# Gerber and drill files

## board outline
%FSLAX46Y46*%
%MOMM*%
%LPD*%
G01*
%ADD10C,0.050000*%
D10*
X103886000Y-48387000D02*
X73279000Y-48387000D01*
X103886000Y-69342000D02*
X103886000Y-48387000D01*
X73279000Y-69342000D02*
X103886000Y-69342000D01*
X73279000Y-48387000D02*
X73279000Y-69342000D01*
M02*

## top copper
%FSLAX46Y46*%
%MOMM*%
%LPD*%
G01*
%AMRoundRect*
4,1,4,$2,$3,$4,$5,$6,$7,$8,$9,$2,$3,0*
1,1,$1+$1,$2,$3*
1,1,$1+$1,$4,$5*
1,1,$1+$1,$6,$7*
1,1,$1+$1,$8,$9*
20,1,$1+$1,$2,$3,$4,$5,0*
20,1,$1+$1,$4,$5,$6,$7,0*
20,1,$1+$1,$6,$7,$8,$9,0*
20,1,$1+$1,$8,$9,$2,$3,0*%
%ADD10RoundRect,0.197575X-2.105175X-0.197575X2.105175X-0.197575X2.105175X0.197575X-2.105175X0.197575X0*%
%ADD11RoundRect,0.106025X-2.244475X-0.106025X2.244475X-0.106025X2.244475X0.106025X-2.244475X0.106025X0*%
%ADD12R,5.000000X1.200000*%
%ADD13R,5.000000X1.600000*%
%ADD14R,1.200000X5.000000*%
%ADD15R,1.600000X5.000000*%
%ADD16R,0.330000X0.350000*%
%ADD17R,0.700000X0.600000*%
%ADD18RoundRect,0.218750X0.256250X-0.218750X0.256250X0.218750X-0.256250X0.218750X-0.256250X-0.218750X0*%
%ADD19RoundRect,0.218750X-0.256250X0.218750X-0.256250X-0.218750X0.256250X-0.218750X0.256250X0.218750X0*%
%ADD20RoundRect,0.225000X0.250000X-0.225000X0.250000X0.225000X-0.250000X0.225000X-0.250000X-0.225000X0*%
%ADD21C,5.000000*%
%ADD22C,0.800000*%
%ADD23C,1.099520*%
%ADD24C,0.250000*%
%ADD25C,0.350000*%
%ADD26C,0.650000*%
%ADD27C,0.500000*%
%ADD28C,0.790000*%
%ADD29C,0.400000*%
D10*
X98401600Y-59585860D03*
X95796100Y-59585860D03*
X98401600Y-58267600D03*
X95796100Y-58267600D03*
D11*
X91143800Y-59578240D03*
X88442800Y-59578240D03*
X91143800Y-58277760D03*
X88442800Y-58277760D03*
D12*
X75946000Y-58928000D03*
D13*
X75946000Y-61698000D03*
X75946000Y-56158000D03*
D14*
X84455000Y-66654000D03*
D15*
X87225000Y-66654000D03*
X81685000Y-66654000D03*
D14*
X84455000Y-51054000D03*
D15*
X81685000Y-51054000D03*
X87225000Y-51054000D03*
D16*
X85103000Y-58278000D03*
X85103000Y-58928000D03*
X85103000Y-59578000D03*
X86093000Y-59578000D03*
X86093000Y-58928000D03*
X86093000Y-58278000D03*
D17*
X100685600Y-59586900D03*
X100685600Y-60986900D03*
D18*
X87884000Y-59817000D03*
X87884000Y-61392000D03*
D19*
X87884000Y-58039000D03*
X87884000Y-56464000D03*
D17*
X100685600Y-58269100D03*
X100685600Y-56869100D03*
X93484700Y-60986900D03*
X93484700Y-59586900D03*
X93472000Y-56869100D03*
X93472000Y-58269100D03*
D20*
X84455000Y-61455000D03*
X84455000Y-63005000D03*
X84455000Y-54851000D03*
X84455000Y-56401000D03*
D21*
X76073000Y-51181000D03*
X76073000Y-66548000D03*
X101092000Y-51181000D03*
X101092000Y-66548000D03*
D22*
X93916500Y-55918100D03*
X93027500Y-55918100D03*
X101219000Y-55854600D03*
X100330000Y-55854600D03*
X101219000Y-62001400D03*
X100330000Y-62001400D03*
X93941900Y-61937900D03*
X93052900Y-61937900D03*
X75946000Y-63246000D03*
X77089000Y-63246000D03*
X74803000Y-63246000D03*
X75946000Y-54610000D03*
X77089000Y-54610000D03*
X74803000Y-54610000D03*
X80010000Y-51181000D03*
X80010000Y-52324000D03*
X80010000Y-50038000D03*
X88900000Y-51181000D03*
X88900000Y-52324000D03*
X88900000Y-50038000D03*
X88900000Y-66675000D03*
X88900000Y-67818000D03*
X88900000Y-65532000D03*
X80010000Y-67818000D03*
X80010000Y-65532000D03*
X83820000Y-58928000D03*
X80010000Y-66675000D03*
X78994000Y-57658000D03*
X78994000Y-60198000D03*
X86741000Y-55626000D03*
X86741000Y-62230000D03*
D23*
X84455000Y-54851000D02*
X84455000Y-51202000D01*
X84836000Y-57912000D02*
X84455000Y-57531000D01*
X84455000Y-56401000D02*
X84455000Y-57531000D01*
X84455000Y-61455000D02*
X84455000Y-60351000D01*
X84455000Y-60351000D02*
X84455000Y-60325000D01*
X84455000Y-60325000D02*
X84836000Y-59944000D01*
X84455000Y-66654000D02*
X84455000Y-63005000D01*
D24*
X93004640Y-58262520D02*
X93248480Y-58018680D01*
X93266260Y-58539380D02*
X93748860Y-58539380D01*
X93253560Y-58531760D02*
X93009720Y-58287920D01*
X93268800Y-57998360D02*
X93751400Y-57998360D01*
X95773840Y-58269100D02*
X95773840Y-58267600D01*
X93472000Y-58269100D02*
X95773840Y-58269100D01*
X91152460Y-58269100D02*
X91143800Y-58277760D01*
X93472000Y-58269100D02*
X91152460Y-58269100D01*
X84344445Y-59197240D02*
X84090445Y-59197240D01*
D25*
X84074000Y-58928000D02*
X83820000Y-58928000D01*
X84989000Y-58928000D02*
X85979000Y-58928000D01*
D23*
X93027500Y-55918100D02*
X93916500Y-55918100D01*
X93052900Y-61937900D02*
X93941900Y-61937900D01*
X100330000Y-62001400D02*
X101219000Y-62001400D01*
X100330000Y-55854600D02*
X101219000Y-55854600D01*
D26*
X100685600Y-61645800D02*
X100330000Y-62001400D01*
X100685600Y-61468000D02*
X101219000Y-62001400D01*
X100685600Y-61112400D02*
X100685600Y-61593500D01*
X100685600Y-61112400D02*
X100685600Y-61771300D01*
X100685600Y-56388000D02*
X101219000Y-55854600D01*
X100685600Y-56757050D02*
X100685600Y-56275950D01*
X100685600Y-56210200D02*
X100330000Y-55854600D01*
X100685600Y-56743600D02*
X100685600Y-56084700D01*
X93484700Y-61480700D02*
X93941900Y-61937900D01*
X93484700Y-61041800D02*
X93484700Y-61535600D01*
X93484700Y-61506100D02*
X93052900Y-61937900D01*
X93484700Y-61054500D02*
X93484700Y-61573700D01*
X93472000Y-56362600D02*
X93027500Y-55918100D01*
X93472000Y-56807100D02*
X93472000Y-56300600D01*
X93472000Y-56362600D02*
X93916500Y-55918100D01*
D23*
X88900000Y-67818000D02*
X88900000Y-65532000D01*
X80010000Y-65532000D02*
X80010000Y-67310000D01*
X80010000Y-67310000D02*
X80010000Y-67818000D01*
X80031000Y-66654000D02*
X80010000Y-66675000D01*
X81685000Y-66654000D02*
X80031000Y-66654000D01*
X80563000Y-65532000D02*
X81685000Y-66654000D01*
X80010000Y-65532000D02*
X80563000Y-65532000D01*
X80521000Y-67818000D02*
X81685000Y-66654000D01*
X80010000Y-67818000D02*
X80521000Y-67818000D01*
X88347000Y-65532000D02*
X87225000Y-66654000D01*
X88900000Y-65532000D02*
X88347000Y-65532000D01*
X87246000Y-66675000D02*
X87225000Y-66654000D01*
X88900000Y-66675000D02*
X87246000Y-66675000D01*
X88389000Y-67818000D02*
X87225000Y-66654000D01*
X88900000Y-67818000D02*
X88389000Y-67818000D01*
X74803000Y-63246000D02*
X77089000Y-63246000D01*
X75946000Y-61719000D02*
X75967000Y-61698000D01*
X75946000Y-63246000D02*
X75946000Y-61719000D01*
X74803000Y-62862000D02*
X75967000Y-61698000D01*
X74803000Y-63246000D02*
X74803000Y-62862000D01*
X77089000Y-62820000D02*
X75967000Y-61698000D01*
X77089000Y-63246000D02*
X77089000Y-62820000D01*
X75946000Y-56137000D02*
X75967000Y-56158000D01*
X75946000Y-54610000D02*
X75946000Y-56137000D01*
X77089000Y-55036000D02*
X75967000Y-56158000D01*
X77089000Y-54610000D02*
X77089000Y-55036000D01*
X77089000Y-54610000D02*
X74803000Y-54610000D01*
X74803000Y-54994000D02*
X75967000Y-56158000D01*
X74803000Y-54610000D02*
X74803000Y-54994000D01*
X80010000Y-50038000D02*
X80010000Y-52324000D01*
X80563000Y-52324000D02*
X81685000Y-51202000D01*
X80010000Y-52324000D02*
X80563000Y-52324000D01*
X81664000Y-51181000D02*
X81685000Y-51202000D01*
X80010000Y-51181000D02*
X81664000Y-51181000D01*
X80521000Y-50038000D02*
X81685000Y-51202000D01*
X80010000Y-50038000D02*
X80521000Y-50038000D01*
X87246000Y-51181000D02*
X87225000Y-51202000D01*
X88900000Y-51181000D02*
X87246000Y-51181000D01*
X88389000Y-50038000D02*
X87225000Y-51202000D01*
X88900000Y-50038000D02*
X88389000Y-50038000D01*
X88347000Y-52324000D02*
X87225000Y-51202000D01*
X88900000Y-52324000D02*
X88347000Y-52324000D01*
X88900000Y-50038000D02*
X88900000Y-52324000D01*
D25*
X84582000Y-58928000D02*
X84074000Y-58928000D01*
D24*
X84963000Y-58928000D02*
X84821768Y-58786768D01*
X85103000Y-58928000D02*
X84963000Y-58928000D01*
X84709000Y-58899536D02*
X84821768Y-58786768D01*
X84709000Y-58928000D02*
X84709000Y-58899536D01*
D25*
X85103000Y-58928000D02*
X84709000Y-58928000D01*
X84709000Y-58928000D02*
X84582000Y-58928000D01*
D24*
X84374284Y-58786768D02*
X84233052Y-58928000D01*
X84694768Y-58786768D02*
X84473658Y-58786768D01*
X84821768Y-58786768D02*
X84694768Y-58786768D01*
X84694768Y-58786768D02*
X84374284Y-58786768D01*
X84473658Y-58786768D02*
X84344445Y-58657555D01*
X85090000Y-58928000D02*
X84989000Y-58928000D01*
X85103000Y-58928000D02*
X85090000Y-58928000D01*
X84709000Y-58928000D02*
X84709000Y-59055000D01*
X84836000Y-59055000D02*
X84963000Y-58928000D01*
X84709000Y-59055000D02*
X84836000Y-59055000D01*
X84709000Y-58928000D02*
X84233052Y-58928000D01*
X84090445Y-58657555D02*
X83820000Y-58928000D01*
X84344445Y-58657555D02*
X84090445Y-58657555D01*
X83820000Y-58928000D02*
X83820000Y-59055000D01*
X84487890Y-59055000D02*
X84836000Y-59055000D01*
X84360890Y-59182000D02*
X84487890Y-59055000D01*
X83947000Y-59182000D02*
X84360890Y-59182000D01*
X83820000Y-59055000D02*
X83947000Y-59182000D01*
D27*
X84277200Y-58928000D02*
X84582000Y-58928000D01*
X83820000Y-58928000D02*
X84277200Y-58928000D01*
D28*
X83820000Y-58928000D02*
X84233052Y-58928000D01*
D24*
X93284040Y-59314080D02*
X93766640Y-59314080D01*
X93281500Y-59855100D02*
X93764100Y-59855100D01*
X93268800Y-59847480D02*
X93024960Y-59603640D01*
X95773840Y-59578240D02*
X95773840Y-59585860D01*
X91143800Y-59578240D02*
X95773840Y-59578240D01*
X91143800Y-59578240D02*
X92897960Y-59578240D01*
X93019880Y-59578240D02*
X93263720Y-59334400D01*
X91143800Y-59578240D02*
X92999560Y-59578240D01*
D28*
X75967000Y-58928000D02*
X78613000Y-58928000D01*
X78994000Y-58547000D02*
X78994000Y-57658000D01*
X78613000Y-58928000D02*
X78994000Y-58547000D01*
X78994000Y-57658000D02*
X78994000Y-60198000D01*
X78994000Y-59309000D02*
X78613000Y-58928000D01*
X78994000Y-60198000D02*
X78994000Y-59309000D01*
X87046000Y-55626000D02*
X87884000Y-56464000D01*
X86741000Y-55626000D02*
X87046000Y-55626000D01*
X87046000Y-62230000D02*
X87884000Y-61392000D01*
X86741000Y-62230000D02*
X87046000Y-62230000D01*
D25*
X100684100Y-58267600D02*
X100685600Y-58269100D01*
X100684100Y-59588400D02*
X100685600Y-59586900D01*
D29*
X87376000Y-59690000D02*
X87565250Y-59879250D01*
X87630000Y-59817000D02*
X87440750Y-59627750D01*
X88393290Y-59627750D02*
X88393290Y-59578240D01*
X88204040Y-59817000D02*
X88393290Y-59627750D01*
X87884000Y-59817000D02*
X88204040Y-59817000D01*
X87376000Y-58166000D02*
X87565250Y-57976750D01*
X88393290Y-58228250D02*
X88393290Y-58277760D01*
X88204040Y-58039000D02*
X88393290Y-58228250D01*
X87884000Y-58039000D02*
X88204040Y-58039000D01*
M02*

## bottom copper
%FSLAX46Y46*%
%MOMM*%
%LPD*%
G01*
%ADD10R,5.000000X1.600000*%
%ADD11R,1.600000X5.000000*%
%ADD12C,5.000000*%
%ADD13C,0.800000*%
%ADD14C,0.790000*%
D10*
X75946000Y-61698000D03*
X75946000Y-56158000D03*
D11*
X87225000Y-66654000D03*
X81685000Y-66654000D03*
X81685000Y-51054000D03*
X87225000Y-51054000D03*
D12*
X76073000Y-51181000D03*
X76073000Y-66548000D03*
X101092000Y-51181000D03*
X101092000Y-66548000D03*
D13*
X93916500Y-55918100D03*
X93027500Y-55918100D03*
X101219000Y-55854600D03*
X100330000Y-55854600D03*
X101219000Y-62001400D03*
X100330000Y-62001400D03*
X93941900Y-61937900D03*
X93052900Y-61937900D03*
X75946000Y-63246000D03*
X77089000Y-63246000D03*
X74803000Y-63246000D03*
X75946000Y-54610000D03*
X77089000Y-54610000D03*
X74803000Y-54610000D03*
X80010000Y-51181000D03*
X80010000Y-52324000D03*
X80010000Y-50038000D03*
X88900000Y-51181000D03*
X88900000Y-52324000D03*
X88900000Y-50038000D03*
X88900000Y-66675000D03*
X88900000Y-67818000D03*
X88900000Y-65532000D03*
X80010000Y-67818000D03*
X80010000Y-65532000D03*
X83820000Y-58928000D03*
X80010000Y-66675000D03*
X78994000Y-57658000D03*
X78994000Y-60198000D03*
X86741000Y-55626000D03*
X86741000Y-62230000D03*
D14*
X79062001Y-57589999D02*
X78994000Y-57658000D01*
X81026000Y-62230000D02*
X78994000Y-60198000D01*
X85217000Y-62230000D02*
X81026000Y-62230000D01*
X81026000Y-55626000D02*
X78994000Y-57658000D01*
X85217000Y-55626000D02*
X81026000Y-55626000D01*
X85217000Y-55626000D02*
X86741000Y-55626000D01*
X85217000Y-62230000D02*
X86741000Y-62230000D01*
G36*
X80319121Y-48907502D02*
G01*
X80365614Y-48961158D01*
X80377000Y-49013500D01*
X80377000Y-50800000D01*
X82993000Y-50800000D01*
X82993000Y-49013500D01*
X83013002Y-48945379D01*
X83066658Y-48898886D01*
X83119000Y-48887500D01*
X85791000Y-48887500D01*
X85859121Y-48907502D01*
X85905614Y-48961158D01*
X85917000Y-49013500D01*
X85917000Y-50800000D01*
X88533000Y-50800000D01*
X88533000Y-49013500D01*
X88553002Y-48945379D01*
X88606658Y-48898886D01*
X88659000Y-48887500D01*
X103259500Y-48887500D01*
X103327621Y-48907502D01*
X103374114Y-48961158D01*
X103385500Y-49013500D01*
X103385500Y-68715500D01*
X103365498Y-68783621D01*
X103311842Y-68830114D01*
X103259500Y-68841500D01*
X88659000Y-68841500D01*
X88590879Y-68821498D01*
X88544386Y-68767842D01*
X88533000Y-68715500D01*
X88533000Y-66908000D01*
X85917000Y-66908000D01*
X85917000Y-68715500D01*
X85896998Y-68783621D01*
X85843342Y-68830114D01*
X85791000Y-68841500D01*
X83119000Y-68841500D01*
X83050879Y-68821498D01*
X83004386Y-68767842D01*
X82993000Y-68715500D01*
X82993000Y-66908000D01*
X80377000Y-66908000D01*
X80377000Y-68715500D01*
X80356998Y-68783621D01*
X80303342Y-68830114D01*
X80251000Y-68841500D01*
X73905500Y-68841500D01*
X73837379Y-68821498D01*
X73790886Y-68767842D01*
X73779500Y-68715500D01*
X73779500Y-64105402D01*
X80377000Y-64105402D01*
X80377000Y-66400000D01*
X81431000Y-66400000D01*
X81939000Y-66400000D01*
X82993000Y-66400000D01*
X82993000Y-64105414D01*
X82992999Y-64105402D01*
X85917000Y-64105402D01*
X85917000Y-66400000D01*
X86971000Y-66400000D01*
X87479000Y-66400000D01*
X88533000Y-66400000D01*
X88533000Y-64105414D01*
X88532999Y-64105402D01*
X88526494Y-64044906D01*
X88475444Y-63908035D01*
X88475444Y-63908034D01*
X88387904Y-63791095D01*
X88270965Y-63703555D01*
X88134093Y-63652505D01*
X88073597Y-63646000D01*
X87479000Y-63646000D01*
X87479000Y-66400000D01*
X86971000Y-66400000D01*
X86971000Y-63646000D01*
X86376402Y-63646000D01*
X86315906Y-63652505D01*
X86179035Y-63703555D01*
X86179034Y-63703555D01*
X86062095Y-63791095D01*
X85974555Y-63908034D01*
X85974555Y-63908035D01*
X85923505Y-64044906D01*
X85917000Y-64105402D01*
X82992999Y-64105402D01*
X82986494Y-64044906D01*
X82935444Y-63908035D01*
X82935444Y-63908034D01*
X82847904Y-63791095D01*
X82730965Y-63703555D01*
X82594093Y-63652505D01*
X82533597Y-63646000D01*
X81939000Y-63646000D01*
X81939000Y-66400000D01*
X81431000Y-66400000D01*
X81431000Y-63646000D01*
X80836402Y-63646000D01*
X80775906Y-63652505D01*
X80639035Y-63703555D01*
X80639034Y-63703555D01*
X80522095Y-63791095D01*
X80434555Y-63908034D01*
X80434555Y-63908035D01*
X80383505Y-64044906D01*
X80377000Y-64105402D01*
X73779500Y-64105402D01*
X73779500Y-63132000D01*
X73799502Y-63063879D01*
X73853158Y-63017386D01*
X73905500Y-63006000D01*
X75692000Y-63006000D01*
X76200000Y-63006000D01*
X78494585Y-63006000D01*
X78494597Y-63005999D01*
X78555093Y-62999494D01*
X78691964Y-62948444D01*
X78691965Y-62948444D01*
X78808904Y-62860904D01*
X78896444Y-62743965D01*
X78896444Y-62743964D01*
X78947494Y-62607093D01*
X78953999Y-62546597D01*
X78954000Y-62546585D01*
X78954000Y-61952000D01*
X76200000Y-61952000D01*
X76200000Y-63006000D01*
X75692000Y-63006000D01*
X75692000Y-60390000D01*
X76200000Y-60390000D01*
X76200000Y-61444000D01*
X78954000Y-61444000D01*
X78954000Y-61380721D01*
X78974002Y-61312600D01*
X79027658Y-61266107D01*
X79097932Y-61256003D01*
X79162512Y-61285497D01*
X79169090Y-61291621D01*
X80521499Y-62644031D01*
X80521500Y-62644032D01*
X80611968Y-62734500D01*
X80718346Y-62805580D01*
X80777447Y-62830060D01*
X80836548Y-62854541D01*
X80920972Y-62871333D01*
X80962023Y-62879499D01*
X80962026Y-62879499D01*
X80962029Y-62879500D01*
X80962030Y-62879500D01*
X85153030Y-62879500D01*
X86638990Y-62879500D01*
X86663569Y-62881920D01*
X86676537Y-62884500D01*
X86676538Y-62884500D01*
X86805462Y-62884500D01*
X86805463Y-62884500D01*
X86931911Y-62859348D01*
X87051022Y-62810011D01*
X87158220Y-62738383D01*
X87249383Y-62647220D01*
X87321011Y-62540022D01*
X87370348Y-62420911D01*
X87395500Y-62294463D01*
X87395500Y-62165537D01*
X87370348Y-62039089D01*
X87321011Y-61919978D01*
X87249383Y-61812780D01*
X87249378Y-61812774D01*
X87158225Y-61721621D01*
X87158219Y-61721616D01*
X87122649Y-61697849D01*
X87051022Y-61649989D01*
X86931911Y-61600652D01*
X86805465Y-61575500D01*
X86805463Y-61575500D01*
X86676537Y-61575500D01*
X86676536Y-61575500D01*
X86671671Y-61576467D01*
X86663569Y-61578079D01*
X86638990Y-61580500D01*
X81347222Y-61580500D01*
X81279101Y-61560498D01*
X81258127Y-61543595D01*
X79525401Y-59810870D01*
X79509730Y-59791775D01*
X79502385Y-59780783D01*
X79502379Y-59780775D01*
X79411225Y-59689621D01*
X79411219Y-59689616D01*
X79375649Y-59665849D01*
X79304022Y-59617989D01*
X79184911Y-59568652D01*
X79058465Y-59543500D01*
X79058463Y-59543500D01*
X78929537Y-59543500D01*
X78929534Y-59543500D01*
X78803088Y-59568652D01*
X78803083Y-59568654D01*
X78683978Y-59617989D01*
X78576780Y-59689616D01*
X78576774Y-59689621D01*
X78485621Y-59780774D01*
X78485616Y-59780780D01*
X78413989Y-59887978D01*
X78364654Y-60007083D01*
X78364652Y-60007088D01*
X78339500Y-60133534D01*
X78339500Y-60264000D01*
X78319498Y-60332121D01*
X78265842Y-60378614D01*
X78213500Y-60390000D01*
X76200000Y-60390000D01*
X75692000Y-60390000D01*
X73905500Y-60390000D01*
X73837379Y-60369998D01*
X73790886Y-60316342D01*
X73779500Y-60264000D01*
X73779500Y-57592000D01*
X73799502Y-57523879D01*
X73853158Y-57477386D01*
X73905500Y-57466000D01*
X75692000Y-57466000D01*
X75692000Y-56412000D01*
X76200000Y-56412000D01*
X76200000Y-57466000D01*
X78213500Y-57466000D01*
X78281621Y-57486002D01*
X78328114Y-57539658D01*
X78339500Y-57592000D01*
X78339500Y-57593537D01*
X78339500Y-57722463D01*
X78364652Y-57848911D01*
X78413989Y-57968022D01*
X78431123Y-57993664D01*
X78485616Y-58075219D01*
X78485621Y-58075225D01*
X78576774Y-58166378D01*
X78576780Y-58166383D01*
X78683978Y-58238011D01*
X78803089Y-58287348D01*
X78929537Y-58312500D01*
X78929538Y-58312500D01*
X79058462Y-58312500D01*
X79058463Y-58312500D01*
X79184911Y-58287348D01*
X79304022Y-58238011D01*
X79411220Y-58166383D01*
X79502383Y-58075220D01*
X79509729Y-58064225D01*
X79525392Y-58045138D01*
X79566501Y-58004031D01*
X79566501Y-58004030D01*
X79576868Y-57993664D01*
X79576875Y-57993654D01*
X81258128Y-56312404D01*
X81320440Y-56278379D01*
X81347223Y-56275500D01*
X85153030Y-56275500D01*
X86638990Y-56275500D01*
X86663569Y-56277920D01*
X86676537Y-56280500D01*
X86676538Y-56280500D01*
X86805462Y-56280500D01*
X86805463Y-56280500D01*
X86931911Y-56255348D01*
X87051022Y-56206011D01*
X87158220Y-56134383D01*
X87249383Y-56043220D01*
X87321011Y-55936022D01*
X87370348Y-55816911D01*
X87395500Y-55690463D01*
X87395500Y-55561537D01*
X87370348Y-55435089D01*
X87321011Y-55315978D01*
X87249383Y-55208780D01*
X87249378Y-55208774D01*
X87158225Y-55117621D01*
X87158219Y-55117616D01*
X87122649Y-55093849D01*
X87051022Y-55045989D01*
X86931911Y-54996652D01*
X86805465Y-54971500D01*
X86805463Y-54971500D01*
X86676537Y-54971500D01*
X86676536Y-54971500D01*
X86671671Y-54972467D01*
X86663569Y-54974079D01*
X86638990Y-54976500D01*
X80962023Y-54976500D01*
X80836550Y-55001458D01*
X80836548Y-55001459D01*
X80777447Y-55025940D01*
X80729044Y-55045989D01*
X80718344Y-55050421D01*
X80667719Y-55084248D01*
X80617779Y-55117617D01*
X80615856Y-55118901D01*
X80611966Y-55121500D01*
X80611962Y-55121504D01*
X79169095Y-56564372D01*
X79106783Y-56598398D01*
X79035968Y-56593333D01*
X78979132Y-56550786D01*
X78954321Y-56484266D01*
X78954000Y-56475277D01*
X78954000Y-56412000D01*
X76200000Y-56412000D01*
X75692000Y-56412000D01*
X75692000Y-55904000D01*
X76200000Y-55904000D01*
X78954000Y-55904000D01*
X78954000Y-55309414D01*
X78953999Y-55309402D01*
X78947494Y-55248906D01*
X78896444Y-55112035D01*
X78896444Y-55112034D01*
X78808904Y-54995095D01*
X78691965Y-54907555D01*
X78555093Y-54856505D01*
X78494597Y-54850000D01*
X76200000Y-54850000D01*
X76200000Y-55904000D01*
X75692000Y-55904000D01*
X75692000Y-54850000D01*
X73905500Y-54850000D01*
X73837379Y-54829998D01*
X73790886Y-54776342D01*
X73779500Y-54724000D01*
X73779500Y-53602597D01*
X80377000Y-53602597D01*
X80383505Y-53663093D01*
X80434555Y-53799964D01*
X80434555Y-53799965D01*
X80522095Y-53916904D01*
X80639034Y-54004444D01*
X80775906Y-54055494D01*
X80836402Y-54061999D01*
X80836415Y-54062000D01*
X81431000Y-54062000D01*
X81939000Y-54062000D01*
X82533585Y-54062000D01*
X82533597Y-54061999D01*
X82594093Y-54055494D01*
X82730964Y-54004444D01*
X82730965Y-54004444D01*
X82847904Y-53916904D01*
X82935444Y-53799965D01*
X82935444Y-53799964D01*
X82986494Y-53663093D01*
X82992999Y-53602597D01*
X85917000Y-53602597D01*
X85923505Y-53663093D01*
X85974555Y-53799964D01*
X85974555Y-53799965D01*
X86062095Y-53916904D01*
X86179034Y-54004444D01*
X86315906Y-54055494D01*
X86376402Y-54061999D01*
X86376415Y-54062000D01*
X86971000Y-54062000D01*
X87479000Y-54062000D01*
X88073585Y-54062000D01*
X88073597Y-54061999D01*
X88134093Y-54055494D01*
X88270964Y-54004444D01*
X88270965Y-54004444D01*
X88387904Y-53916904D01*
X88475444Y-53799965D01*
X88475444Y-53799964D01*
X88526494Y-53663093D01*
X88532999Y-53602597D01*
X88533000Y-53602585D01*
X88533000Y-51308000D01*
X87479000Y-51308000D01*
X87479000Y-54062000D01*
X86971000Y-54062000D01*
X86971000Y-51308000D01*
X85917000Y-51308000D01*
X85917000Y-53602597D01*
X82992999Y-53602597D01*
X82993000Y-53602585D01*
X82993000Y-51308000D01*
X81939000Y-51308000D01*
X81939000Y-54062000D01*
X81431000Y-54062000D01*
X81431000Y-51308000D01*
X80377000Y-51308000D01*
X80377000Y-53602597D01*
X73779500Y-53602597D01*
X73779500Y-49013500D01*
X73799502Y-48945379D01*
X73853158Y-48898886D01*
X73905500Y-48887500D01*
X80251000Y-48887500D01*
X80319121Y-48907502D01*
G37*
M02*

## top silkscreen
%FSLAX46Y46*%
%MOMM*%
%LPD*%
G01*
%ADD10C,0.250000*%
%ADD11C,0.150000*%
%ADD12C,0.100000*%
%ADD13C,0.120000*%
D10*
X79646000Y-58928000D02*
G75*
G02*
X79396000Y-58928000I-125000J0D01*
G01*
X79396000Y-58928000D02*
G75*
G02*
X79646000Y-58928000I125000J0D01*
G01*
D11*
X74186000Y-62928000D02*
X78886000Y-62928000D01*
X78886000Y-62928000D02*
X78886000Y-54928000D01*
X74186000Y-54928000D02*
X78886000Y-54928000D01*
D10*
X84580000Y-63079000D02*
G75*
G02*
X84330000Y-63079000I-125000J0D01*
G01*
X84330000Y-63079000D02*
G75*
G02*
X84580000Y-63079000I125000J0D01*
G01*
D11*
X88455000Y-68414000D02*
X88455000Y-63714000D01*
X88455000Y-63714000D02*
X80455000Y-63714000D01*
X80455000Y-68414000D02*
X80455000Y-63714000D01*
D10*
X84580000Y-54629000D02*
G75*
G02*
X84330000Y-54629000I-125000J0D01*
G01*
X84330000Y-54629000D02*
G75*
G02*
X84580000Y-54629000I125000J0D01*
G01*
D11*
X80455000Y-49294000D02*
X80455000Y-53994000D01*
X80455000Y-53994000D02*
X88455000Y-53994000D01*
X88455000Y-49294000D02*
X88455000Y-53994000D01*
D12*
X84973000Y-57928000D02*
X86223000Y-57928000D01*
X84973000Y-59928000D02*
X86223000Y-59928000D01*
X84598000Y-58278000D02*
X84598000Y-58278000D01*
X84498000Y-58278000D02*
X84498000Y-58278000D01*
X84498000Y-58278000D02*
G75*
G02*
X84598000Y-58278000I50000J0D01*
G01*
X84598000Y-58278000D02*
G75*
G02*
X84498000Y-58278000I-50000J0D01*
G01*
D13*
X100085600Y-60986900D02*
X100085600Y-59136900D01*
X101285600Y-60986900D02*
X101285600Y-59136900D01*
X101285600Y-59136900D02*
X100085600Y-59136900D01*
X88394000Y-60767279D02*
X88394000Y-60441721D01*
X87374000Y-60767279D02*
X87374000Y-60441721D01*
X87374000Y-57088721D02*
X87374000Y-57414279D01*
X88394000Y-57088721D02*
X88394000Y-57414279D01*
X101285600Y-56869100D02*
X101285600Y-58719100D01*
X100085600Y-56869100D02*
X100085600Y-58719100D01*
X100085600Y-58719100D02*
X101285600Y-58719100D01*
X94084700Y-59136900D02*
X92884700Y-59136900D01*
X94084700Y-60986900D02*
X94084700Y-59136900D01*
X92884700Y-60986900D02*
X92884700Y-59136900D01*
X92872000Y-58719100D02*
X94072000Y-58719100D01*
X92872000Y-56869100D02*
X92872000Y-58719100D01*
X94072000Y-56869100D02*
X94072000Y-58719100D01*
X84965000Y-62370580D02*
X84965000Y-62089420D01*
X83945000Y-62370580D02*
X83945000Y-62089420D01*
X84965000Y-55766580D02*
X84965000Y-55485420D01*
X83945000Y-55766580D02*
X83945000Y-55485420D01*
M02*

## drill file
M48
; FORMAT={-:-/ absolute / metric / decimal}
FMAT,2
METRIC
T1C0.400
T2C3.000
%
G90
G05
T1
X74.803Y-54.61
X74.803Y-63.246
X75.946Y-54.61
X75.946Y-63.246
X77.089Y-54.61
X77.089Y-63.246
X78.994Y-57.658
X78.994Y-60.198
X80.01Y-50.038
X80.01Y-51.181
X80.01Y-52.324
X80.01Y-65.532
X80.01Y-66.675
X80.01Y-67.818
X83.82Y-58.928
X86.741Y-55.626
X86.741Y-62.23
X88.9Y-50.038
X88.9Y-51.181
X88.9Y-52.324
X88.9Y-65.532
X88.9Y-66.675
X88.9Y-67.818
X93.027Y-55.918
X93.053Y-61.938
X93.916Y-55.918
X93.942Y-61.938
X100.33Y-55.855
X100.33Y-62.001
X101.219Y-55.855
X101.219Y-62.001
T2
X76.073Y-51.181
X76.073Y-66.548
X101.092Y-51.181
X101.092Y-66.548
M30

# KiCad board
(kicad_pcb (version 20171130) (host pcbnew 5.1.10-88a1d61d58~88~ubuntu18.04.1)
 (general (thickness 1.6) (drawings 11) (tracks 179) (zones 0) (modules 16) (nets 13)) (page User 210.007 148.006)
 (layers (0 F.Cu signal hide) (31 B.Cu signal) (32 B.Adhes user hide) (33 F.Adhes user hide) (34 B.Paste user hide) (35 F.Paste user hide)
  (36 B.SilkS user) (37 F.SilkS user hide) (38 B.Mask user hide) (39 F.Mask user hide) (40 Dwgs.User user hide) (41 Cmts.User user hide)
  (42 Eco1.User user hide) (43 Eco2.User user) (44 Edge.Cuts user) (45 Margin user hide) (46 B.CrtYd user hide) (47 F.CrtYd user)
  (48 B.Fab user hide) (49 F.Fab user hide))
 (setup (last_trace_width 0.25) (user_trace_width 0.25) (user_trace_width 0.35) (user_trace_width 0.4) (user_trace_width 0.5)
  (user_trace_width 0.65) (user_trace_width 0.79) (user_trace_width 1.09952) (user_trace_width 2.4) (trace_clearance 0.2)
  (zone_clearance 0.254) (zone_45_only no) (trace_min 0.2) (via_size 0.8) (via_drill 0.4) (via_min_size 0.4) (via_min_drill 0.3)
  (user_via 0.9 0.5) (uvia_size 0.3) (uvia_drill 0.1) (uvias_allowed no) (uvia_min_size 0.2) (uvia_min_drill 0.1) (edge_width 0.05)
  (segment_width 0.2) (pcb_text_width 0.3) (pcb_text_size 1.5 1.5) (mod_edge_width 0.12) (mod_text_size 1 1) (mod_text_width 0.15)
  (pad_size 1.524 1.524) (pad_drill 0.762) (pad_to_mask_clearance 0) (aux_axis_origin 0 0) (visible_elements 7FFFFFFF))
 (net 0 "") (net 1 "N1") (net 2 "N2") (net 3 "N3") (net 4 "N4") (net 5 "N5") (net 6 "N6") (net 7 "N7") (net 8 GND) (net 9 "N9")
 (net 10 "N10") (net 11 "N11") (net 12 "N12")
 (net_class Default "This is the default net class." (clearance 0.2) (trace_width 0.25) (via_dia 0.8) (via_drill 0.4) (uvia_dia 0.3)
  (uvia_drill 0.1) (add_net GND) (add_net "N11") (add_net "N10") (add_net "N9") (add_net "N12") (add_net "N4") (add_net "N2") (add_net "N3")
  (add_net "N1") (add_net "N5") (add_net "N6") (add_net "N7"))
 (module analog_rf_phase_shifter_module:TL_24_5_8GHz (layer F.Cu) (at 97.09885 59.58586)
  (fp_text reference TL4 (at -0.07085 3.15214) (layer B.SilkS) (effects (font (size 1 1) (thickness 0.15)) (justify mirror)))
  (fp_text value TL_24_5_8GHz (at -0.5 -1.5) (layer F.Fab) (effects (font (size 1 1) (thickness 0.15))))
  (pad 2 smd roundrect (at 1.30275 0) (size 4.6055 0.7903) (layers F.Cu F.Mask) (roundrect_rratio 0.25) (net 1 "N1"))
  (pad 1 smd roundrect (at -1.30275 0) (size 4.6055 0.7903) (layers F.Cu F.Mask) (roundrect_rratio 0.25) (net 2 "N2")))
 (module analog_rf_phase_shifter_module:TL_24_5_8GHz (layer F.Cu) (at 97.09885 58.2676)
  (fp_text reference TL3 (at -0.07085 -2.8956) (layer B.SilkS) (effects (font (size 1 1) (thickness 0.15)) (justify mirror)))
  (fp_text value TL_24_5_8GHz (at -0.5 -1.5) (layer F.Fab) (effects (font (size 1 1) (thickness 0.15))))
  (pad 2 smd roundrect (at 1.30275 0) (size 4.6055 0.7903) (layers F.Cu F.Mask) (roundrect_rratio 0.25) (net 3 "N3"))
  (pad 1 smd roundrect (at -1.30275 0) (size 4.6055 0.7903) (layers F.Cu F.Mask) (roundrect_rratio 0.25) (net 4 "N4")))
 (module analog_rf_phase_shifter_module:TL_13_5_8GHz (layer F.Cu) (at 89.7933 59.57824)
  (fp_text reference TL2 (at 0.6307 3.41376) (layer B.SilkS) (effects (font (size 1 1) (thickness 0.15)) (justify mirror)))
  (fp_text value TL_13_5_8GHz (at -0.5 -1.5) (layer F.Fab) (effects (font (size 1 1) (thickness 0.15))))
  (pad 2 smd roundrect (at 1.3505 0) (size 4.701 0.4241) (layers F.Cu F.Mask) (roundrect_rratio 0.25) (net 2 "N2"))
  (pad 1 smd roundrect (at -1.3505 0) (size 4.701 0.4241) (layers F.Cu F.Mask) (roundrect_rratio 0.25) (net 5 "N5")))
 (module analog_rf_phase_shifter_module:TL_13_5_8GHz (layer F.Cu) (at 89.7933 58.27776)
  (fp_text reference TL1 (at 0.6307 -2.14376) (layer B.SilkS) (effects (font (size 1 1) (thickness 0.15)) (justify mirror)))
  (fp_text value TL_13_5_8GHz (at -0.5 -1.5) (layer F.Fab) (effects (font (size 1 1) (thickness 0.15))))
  (pad 2 smd roundrect (at 1.3505 0) (size 4.701 0.4241) (layers F.Cu F.Mask) (roundrect_rratio 0.25) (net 4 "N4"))
  (pad 1 smd roundrect (at -1.3505 0) (size 4.701 0.4241) (layers F.Cu F.Mask) (roundrect_rratio 0.25) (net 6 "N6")))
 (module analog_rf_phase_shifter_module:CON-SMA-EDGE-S (layer F.Cu) (at 68.686 58.928 90)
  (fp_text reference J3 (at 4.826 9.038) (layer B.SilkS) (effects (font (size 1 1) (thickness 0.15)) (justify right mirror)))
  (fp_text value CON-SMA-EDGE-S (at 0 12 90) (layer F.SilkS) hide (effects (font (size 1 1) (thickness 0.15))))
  (fp_circle (center 0 10.835) (end 0.125 10.835) (layer F.SilkS) (width 0.25))
  (fp_line (start -4 5.5) (end -4 10.2) (layer F.SilkS) (width 0.15))
  (fp_line (start -4 10.2) (end 4 10.2) (layer F.SilkS) (width 0.15))
  (fp_line (start 4 5.5) (end 4 10.2) (layer F.SilkS) (width 0.15))
  (pad 1 smd rect (at 0 7.26 90) (size 1.2 5) (layers F.Cu F.Paste F.Mask) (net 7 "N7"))
  (pad 2 smd rect (at -2.77 7.26 90) (size 1.6 5) (layers F.Cu F.Paste F.Mask) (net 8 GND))
  (pad 2 smd rect (at 2.77 7.26 90) (size 1.6 5) (layers F.Cu F.Paste F.Mask) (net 8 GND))
  (pad 2 smd rect (at -2.77 7.26 90) (size 1.6 5) (layers B.Cu B.Paste B.Mask) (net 8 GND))
  (pad 2 smd rect (at 2.77 7.26 90) (size 1.6 5) (layers B.Cu B.Paste B.Mask) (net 8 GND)))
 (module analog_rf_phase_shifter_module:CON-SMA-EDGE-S (layer F.Cu) (at 84.455 73.914 180)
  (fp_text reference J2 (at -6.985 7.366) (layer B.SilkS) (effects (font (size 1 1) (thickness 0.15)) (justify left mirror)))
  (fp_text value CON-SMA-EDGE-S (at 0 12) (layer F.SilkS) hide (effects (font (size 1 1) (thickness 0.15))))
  (fp_circle (center 0 10.835) (end 0.125 10.835) (layer F.SilkS) (width 0.25))
  (fp_line (start -4 5.5) (end -4 10.2) (layer F.SilkS) (width 0.15))
  (fp_line (start -4 10.2) (end 4 10.2) (layer F.SilkS) (width 0.15))
  (fp_line (start 4 5.5) (end 4 10.2) (layer F.SilkS) (width 0.15))
  (pad 1 smd rect (at 0 7.26 180) (size 1.2 5) (layers F.Cu F.Paste F.Mask) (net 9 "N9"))
  (pad 2 smd rect (at -2.77 7.26 180) (size 1.6 5) (layers F.Cu F.Paste F.Mask) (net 8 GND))
  (pad 2 smd rect (at 2.77 7.26 180) (size 1.6 5) (layers F.Cu F.Paste F.Mask) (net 8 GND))
  (pad 2 smd rect (at -2.77 7.26 180) (size 1.6 5) (layers B.Cu B.Paste B.Mask) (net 8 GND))
  (pad 2 smd rect (at 2.77 7.26 180) (size 1.6 5) (layers B.Cu B.Paste B.Mask) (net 8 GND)))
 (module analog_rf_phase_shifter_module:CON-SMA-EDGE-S (layer F.Cu) (at 84.455 43.794)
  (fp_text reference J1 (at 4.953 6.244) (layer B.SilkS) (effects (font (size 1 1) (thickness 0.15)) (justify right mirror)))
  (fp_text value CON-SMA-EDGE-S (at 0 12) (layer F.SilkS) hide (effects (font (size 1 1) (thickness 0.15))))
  (fp_circle (center 0 10.835) (end 0.125 10.835) (layer F.SilkS) (width 0.25))
  (fp_line (start -4 5.5) (end -4 10.2) (layer F.SilkS) (width 0.15))
  (fp_line (start -4 10.2) (end 4 10.2) (layer F.SilkS) (width 0.15))
  (fp_line (start 4 5.5) (end 4 10.2) (layer F.SilkS) (width 0.15))
  (pad 1 smd rect (at 0 7.26) (size 1.2 5) (layers F.Cu F.Paste F.Mask) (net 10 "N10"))
  (pad 2 smd rect (at -2.77 7.26) (size 1.6 5) (layers F.Cu F.Paste F.Mask) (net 8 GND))
  (pad 2 smd rect (at 2.77 7.26) (size 1.6 5) (layers F.Cu F.Paste F.Mask) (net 8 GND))
  (pad 2 smd rect (at -2.77 7.26) (size 1.6 5) (layers B.Cu B.Paste B.Mask) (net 8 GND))
  (pad 2 smd rect (at 2.77 7.26) (size 1.6 5) (layers B.Cu B.Paste B.Mask) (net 8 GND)))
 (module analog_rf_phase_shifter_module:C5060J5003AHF (layer F.Cu) (at 85.598 58.928 270)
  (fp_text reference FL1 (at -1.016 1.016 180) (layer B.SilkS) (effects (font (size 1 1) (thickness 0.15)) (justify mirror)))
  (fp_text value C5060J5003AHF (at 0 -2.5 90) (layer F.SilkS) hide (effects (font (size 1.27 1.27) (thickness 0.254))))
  (fp_line (start -1 0.625) (end -1 -0.625) (layer F.SilkS) (width 0.1))
  (fp_line (start 1 0.625) (end 1 -0.625) (layer F.SilkS) (width 0.1))
  (fp_line (start -0.65 1) (end -0.65 1) (layer F.SilkS) (width 0.1))
  (fp_line (start -0.65 1.1) (end -0.65 1.1) (layer F.SilkS) (width 0.1))
  (fp_arc (start -0.65 1.05) (end -0.65 1) (angle -180) (layer F.SilkS) (width 0.1))
  (fp_arc (start -0.65 1.05) (end -0.65 1.1) (angle -180) (layer F.SilkS) (width 0.1))
  (pad 1 smd rect (at -0.65 0.495) (size 0.33 0.35) (layers F.Cu F.Paste F.Mask) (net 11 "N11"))
  (pad 2 smd rect (at 0 0.495) (size 0.33 0.35) (layers F.Cu F.Paste F.Mask) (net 8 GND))
  (pad 3 smd rect (at 0.65 0.495) (size 0.33 0.35) (layers F.Cu F.Paste F.Mask) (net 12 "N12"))
  (pad 4 smd rect (at 0.65 -0.495) (size 0.33 0.35) (layers F.Cu F.Paste F.Mask) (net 5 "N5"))
  (pad 5 smd rect (at 0 -0.495) (size 0.33 0.35) (layers F.Cu F.Paste F.Mask) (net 8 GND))
  (pad 6 smd rect (at -0.65 -0.495) (size 0.33 0.35) (layers F.Cu F.Paste F.Mask) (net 6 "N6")))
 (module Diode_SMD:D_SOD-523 (layer F.Cu) (at 100.6856 60.2869 270)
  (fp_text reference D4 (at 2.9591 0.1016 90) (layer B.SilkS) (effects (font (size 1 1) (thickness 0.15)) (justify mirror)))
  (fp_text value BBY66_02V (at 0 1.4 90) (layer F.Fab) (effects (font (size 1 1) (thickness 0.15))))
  (fp_line (start 0.7 0.6) (end -1.15 0.6) (layer F.SilkS) (width 0.12))
  (fp_line (start 0.7 -0.6) (end -1.15 -0.6) (layer F.SilkS) (width 0.12))
  (fp_line (start -1.15 -0.6) (end -1.15 0.6) (layer F.SilkS) (width 0.12))
  (pad 1 smd rect (at -0.7 0 90) (size 0.6 0.7) (layers F.Cu F.Paste F.Mask) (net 1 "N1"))
  (pad 2 smd rect (at 0.7 0 90) (size 0.6 0.7) (layers F.Cu F.Paste F.Mask) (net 8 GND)))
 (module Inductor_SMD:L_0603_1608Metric (layer F.Cu) (at 87.884 60.6045 90)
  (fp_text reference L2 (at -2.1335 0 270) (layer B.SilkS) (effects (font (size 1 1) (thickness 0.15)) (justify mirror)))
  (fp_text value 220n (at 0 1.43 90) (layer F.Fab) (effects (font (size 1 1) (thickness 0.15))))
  (fp_line (start -0.162779 0.51) (end 0.162779 0.51) (layer F.SilkS) (width 0.12))
  (fp_line (start -0.162779 -0.51) (end 0.162779 -0.51) (layer F.SilkS) (width 0.12))
  (pad 2 smd roundrect (at 0.7875 0 90) (size 0.875 0.95) (layers F.Cu F.Paste F.Mask) (roundrect_rratio 0.25) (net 5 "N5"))
  (pad 1 smd roundrect (at -0.7875 0 90) (size 0.875 0.95) (layers F.Cu F.Paste F.Mask) (roundrect_rratio 0.25) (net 7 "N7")))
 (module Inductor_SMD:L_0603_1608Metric (layer F.Cu) (at 87.884 57.2515 270)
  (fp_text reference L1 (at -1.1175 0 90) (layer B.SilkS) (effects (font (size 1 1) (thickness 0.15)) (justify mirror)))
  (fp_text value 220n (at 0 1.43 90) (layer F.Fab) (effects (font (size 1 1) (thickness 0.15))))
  (fp_line (start -0.162779 0.51) (end 0.162779 0.51) (layer F.SilkS) (width 0.12))
  (fp_line (start -0.162779 -0.51) (end 0.162779 -0.51) (layer F.SilkS) (width 0.12))
  (pad 2 smd roundrect (at 0.7875 0 270) (size 0.875 0.95) (layers F.Cu F.Paste F.Mask) (roundrect_rratio 0.25) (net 6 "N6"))
  (pad 1 smd roundrect (at -0.7875 0 270) (size 0.875 0.95) (layers F.Cu F.Paste F.Mask) (roundrect_rratio 0.25) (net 7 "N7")))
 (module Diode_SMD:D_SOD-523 (layer F.Cu) (at 100.6856 57.5691 90)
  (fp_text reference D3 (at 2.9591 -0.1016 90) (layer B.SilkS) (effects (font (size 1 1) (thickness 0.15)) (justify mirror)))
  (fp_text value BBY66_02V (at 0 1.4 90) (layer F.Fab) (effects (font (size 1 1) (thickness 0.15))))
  (fp_line (start 0.7 0.6) (end -1.15 0.6) (layer F.SilkS) (width 0.12))
  (fp_line (start 0.7 -0.6) (end -1.15 -0.6) (layer F.SilkS) (width 0.12))
  (fp_line (start -1.15 -0.6) (end -1.15 0.6) (layer F.SilkS) (width 0.12))
  (pad 1 smd rect (at -0.7 0 270) (size 0.6 0.7) (layers F.Cu F.Paste F.Mask) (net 3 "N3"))
  (pad 2 smd rect (at 0.7 0 270) (size 0.6 0.7) (layers F.Cu F.Paste F.Mask) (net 8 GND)))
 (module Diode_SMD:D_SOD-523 (layer F.Cu) (at 93.4847 60.2869 270)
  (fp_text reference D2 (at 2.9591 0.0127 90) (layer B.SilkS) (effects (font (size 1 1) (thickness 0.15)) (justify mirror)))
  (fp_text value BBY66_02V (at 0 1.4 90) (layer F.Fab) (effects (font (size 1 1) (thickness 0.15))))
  (fp_line (start -1.15 -0.6) (end -1.15 0.6) (layer F.SilkS) (width 0.12))
  (fp_line (start 0.7 -0.6) (end -1.15 -0.6) (layer F.SilkS) (width 0.12))
  (fp_line (start 0.7 0.6) (end -1.15 0.6) (layer F.SilkS) (width 0.12))
  (pad 2 smd rect (at 0.7 0 90) (size 0.6 0.7) (layers F.Cu F.Paste F.Mask) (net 8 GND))
  (pad 1 smd rect (at -0.7 0 90) (size 0.6 0.7) (layers F.Cu F.Paste F.Mask) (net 2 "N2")))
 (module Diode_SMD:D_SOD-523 (layer F.Cu) (at 93.472 57.5691 90)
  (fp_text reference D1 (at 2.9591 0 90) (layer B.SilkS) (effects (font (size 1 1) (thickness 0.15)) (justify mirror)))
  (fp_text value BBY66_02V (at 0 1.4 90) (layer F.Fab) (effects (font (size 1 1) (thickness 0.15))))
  (fp_line (start -1.15 -0.6) (end -1.15 0.6) (layer F.SilkS) (width 0.12))
  (fp_line (start 0.7 -0.6) (end -1.15 -0.6) (layer F.SilkS) (width 0.12))
  (fp_line (start 0.7 0.6) (end -1.15 0.6) (layer F.SilkS) (width 0.12))
  (pad 2 smd rect (at 0.7 0 270) (size 0.6 0.7) (layers F.Cu F.Paste F.Mask) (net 8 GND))
  (pad 1 smd rect (at -0.7 0 270) (size 0.6 0.7) (layers F.Cu F.Paste F.Mask) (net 4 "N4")))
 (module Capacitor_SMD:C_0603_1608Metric (layer F.Cu) (at 84.455 62.23 90)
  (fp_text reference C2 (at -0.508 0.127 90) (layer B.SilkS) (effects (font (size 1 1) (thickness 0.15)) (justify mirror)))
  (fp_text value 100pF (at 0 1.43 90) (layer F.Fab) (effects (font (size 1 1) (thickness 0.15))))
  (fp_line (start -0.14058 0.51) (end 0.14058 0.51) (layer F.SilkS) (width 0.12))
  (fp_line (start -0.14058 -0.51) (end 0.14058 -0.51) (layer F.SilkS) (width 0.12))
  (pad 2 smd roundrect (at 0.775 0 90) (size 0.9 0.95) (layers F.Cu F.Paste F.Mask) (roundrect_rratio 0.25) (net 12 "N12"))
  (pad 1 smd roundrect (at -0.775 0 90) (size 0.9 0.95) (layers F.Cu F.Paste F.Mask) (roundrect_rratio 0.25) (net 9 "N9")))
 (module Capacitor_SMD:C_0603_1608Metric (layer F.Cu) (at 84.455 55.626 90)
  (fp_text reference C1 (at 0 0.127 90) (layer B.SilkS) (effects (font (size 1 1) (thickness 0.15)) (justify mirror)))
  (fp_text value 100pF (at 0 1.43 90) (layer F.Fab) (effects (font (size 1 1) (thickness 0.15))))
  (fp_line (start -0.14058 0.51) (end 0.14058 0.51) (layer F.SilkS) (width 0.12))
  (fp_line (start -0.14058 -0.51) (end 0.14058 -0.51) (layer F.SilkS) (width 0.12))
  (pad 2 smd roundrect (at 0.775 0 90) (size 0.9 0.95) (layers F.Cu F.Paste F.Mask) (roundrect_rratio 0.25) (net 10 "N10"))
  (pad 1 smd roundrect (at -0.775 0 90) (size 0.9 0.95) (layers F.Cu F.Paste F.Mask) (roundrect_rratio 0.25) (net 11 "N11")))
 (gr_line (start 103.886 48.387) (end 73.279 48.387) (layer Edge.Cuts) (width 0.05))
 (gr_line (start 103.886 69.342) (end 103.886 48.387) (layer Edge.Cuts) (width 0.05))
 (gr_line (start 73.279 69.342) (end 103.886 69.342) (layer Edge.Cuts) (width 0.05))
 (gr_line (start 73.279 48.387) (end 73.279 69.342) (layer Edge.Cuts) (width 0.05))
 (segment (start 84.455 54.851) (end 84.455 51.202) (width 1.09952) (layer F.Cu) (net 10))
 (segment (start 84.836 57.912) (end 84.455 57.531) (width 1.09952) (layer F.Cu) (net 11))
 (segment (start 84.455 56.401) (end 84.455 57.531) (width 1.09952) (layer F.Cu) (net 11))
 (segment (start 84.455 61.455) (end 84.455 60.351) (width 1.09952) (layer F.Cu) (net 12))
 (segment (start 84.455 60.351) (end 84.455 60.325) (width 1.09952) (layer F.Cu) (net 12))
 (segment (start 84.455 60.325) (end 84.836 59.944) (width 1.09952) (layer F.Cu) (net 12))
 (segment (start 84.455 66.654) (end 84.455 63.005) (width 1.09952) (layer F.Cu) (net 9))
 (segment (start 93.00464 58.26252) (end 93.24848 58.01868) (width 0.25) (layer F.Cu) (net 4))
 (segment (start 93.26626 58.53938) (end 93.74886 58.53938) (width 0.25) (layer F.Cu) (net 4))
 (segment (start 93.25356 58.53176) (end 93.00972 58.28792) (width 0.25) (layer F.Cu) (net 4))
 (segment (start 93.2688 57.99836) (end 93.7514 57.99836) (width 0.25) (layer F.Cu) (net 4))
 (segment (start 95.77384 58.2691) (end 95.77384 58.2676) (width 0.25) (layer F.Cu) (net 4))
 (segment (start 93.472 58.2691) (end 95.77384 58.2691) (width 0.25) (layer F.Cu) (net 4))
 (segment (start 91.15246 58.2691) (end 91.1438 58.27776) (width 0.25) (layer F.Cu) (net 4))
 (segment (start 93.472 58.2691) (end 91.15246 58.2691) (width 0.25) (layer F.Cu) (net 4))
 (segment (start 84.344445 59.19724) (end 84.090445 59.19724) (width 0.25) (layer F.Cu) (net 8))
 (via (at 76.073 51.181) (size 5) (drill 3) (layers F.Cu B.Cu) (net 8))
 (via (at 76.073 66.548) (size 5) (drill 3) (layers F.Cu B.Cu) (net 8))
 (via (at 101.092 51.181) (size 5) (drill 3) (layers F.Cu B.Cu) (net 8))
 (via (at 101.092 66.548) (size 5) (drill 3) (layers F.Cu B.Cu) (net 8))
 (via (at 93.9165 55.9181) (size 0.8) (drill 0.4) (layers F.Cu B.Cu) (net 8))
 (via (at 93.0275 55.9181) (size 0.8) (drill 0.4) (layers F.Cu B.Cu) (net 8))
 (via (at 101.219 55.8546) (size 0.8) (drill 0.4) (layers F.Cu B.Cu) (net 8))
 (via (at 100.33 55.8546) (size 0.8) (drill 0.4) (layers F.Cu B.Cu) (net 8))
 (via (at 101.219 62.0014) (size 0.8) (drill 0.4) (layers F.Cu B.Cu) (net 8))
 (via (at 100.33 62.0014) (size 0.8) (drill 0.4) (layers F.Cu B.Cu) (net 8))
 (via (at 93.9419 61.9379) (size 0.8) (drill 0.4) (layers F.Cu B.Cu) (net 8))
 (via (at 93.0529 61.9379) (size 0.8) (drill 0.4) (layers F.Cu B.Cu) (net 8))
 (via (at 75.946 63.246) (size 0.8) (drill 0.4) (layers F.Cu B.Cu) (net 8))
 (via (at 77.089 63.246) (size 0.8) (drill 0.4) (layers F.Cu B.Cu) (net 8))
 (via (at 74.803 63.246) (size 0.8) (drill 0.4) (layers F.Cu B.Cu) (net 8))
 (via (at 75.946 54.61) (size 0.8) (drill 0.4) (layers F.Cu B.Cu) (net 8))
 (via (at 77.089 54.61) (size 0.8) (drill 0.4) (layers F.Cu B.Cu) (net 8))
 (via (at 74.803 54.61) (size 0.8) (drill 0.4) (layers F.Cu B.Cu) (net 8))
 (via (at 80.01 51.181) (size 0.8) (drill 0.4) (layers F.Cu B.Cu) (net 8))
 (via (at 80.01 52.324) (size 0.8) (drill 0.4) (layers F.Cu B.Cu) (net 8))
 (via (at 80.01 50.038) (size 0.8) (drill 0.4) (layers F.Cu B.Cu) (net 8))
 (via (at 88.9 51.181) (size 0.8) (drill 0.4) (layers F.Cu B.Cu) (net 8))
 (via (at 88.9 52.324) (size 0.8) (drill 0.4) (layers F.Cu B.Cu) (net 8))
 (via (at 88.9 50.038) (size 0.8) (drill 0.4) (layers F.Cu B.Cu) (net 8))
 (via (at 88.9 66.675) (size 0.8) (drill 0.4) (layers F.Cu B.Cu) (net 8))
 (via (at 88.9 67.818) (size 0.8) (drill 0.4) (layers F.Cu B.Cu) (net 8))
 (via (at 88.9 65.532) (size 0.8) (drill 0.4) (layers F.Cu B.Cu) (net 8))
 (via (at 80.01 67.818) (size 0.8) (drill 0.4) (layers F.Cu B.Cu) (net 8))
 (via (at 80.01 65.532) (size 0.8) (drill 0.4) (layers F.Cu B.Cu) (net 8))
 (via (at 83.82 58.928) (size 0.8) (drill 0.4) (layers F.Cu B.Cu) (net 8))
 (segment (start 84.074 58.928) (end 83.82 58.928) (width 0.35) (layer F.Cu) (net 8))
 (segment (start 84.989 58.928) (end 85.979 58.928) (width 0.35) (layer F.Cu) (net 8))
 (via (at 80.01 66.675) (size 0.8) (drill 0.4) (layers F.Cu B.Cu) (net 8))
 (segment (start 93.0275 55.9181) (end 93.9165 55.9181) (width 1.09952) (layer F.Cu) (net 8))
 (segment (start 93.0529 61.9379) (end 93.9419 61.9379) (width 1.09952) (layer F.Cu) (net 8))
 (segment (start 100.33 62.0014) (end 101.219 62.0014) (width 1.09952) (layer F.Cu) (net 8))
 (segment (start 100.33 55.8546) (end 101.219 55.8546) (width 1.09952) (layer F.Cu) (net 8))
 (segment (start 100.6856 61.6458) (end 100.33 62.0014) (width 0.65) (layer F.Cu) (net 8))
 (segment (start 100.6856 61.468) (end 101.219 62.0014) (width 0.65) (layer F.Cu) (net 8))
 (segment (start 100.6856 61.1124) (end 100.6856 61.5935) (width 0.65) (layer F.Cu) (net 8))
 (segment (start 100.6856 61.1124) (end 100.6856 61.7713) (width 0.65) (layer F.Cu) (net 8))
 (segment (start 100.6856 56.388) (end 101.219 55.8546) (width 0.65) (layer F.Cu) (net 8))
 (segment (start 100.6856 56.75705) (end 100.6856 56.27595) (width 0.65) (layer F.Cu) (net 8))
 (segment (start 100.6856 56.2102) (end 100.33 55.8546) (width 0.65) (layer F.Cu) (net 8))
 (segment (start 100.6856 56.7436) (end 100.6856 56.0847) (width 0.65) (layer F.Cu) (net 8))
 (segment (start 93.4847 61.4807) (end 93.9419 61.9379) (width 0.65) (layer F.Cu) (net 8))
 (segment (start 93.4847 61.0418) (end 93.4847 61.5356) (width 0.65) (layer F.Cu) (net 8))
 (segment (start 93.4847 61.5061) (end 93.0529 61.9379) (width 0.65) (layer F.Cu) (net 8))
 (segment (start 93.4847 61.0545) (end 93.4847 61.5737) (width 0.65) (layer F.Cu) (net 8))
 (segment (start 93.472 56.3626) (end 93.0275 55.9181) (width 0.65) (layer F.Cu) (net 8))
 (segment (start 93.472 56.8071) (end 93.472 56.3006) (width 0.65) (layer F.Cu) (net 8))
 (segment (start 93.472 56.3626) (end 93.9165 55.9181) (width 0.65) (layer F.Cu) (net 8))
 (segment (start 88.9 67.818) (end 88.9 65.532) (width 1.09952) (layer F.Cu) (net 8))
 (segment (start 80.01 65.532) (end 80.01 67.31) (width 1.09952) (layer F.Cu) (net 8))
 (segment (start 80.01 67.31) (end 80.01 67.818) (width 1.09952) (layer F.Cu) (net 8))
 (segment (start 80.031 66.654) (end 80.01 66.675) (width 1.09952) (layer F.Cu) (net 8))
 (segment (start 81.685 66.654) (end 80.031 66.654) (width 1.09952) (layer F.Cu) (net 8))
 (segment (start 80.563 65.532) (end 81.685 66.654) (width 1.09952) (layer F.Cu) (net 8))
 (segment (start 80.01 65.532) (end 80.563 65.532) (width 1.09952) (layer F.Cu) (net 8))
 (segment (start 80.521 67.818) (end 81.685 66.654) (width 1.09952) (layer F.Cu) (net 8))
 (segment (start 80.01 67.818) (end 80.521 67.818) (width 1.09952) (layer F.Cu) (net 8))
 (segment (start 88.347 65.532) (end 87.225 66.654) (width 1.09952) (layer F.Cu) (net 8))
 (segment (start 88.9 65.532) (end 88.347 65.532) (width 1.09952) (layer F.Cu) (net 8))
 (segment (start 87.246 66.675) (end 87.225 66.654) (width 1.09952) (layer F.Cu) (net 8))
 (segment (start 88.9 66.675) (end 87.246 66.675) (width 1.09952) (layer F.Cu) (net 8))
 (segment (start 88.389 67.818) (end 87.225 66.654) (width 1.09952) (layer F.Cu) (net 8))
 (segment (start 88.9 67.818) (end 88.389 67.818) (width 1.09952) (layer F.Cu) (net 8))
 (segment (start 74.803 63.246) (end 77.089 63.246) (width 1.09952) (layer F.Cu) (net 8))
 (segment (start 75.946 61.719) (end 75.967 61.698) (width 1.09952) (layer F.Cu) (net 8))
 (segment (start 75.946 63.246) (end 75.946 61.719) (width 1.09952) (layer F.Cu) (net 8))
 (segment (start 74.803 62.862) (end 75.967 61.698) (width 1.09952) (layer F.Cu) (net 8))
 (segment (start 74.803 63.246) (end 74.803 62.862) (width 1.09952) (layer F.Cu) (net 8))
 (segment (start 77.089 62.82) (end 75.967 61.698) (width 1.09952) (layer F.Cu) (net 8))
 (segment (start 77.089 63.246) (end 77.089 62.82) (width 1.09952) (layer F.Cu) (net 8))
 (segment (start 75.946 56.137) (end 75.967 56.158) (width 1.09952) (layer F.Cu) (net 8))
 (segment (start 75.946 54.61) (end 75.946 56.137) (width 1.09952) (layer F.Cu) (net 8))
 (segment (start 77.089 55.036) (end 75.967 56.158) (width 1.09952) (layer F.Cu) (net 8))
 (segment (start 77.089 54.61) (end 77.089 55.036) (width 1.09952) (layer F.Cu) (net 8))
 (segment (start 77.089 54.61) (end 74.803 54.61) (width 1.09952) (layer F.Cu) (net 8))
 (segment (start 74.803 54.994) (end 75.967 56.158) (width 1.09952) (layer F.Cu) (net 8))
 (segment (start 74.803 54.61) (end 74.803 54.994) (width 1.09952) (layer F.Cu) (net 8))
 (segment (start 80.01 50.038) (end 80.01 52.324) (width 1.09952) (layer F.Cu) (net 8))
 (segment (start 80.563 52.324) (end 81.685 51.202) (width 1.09952) (layer F.Cu) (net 8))
 (segment (start 80.01 52.324) (end 80.563 52.324) (width 1.09952) (layer F.Cu) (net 8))
 (segment (start 81.664 51.181) (end 81.685 51.202) (width 1.09952) (layer F.Cu) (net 8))
 (segment (start 80.01 51.181) (end 81.664 51.181) (width 1.09952) (layer F.Cu) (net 8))
 (segment (start 80.521 50.038) (end 81.685 51.202) (width 1.09952) (layer F.Cu) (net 8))
 (segment (start 80.01 50.038) (end 80.521 50.038) (width 1.09952) (layer F.Cu) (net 8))
 (segment (start 87.246 51.181) (end 87.225 51.202) (width 1.09952) (layer F.Cu) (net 8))
 (segment (start 88.9 51.181) (end 87.246 51.181) (width 1.09952) (layer F.Cu) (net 8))
 (segment (start 88.389 50.038) (end 87.225 51.202) (width 1.09952) (layer F.Cu) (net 8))
 (segment (start 88.9 50.038) (end 88.389 50.038) (width 1.09952) (layer F.Cu) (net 8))
 (segment (start 88.347 52.324) (end 87.225 51.202) (width 1.09952) (layer F.Cu) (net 8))
 (segment (start 88.9 52.324) (end 88.347 52.324) (width 1.09952) (layer F.Cu) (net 8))
 (segment (start 88.9 50.038) (end 88.9 52.324) (width 1.09952) (layer F.Cu) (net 8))
 (segment (start 84.582 58.928) (end 84.074 58.928) (width 0.35) (layer F.Cu) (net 8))
 (segment (start 84.963 58.928) (end 84.821768 58.786768) (width 0.25) (layer F.Cu) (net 8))
 (segment (start 85.103 58.928) (end 84.963 58.928) (width 0.25) (layer F.Cu) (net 8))
 (segment (start 84.709 58.899536) (end 84.821768 58.786768) (width 0.25) (layer F.Cu) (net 8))
 (segment (start 84.709 58.928) (end 84.709 58.899536) (width 0.25) (layer F.Cu) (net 8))
 (segment (start 85.103 58.928) (end 84.709 58.928) (width 0.35) (layer F.Cu) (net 8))
 (segment (start 84.709 58.928) (end 84.582 58.928) (width 0.35) (layer F.Cu) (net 8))
 (segment (start 84.374284 58.786768) (end 84.233052 58.928) (width 0.25) (layer F.Cu) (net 8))
 (segment (start 84.694768 58.786768) (end 84.473658 58.786768) (width 0.25) (layer F.Cu) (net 8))
 (segment (start 84.821768 58.786768) (end 84.694768 58.786768) (width 0.25) (layer F.Cu) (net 8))
 (segment (start 84.694768 58.786768) (end 84.374284 58.786768) (width 0.25) (layer F.Cu) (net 8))
 (segment (start 84.473658 58.786768) (end 84.344445 58.657555) (width 0.25) (layer F.Cu) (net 8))
 (segment (start 85.09 58.928) (end 84.989 58.928) (width 0.25) (layer F.Cu) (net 8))
 (segment (start 85.103 58.928) (end 85.09 58.928) (width 0.25) (layer F.Cu) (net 8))
 (segment (start 84.709 58.928) (end 84.709 59.055) (width 0.25) (layer F.Cu) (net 8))
 (segment (start 84.836 59.055) (end 84.963 58.928) (width 0.25) (layer F.Cu) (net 8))
 (segment (start 84.709 59.055) (end 84.836 59.055) (width 0.25) (layer F.Cu) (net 8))
 (segment (start 84.709 58.928) (end 84.233052 58.928) (width 0.25) (layer F.Cu) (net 8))
 (segment (start 84.090445 58.657555) (end 83.82 58.928) (width 0.25) (layer F.Cu) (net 8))
 (segment (start 84.344445 58.657555) (end 84.090445 58.657555) (width 0.25) (layer F.Cu) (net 8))
 (segment (start 83.82 58.928) (end 83.82 59.055) (width 0.25) (layer F.Cu) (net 8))
 (segment (start 84.48789 59.055) (end 84.836 59.055) (width 0.25) (layer F.Cu) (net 8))
 (segment (start 84.36089 59.182) (end 84.48789 59.055) (width 0.25) (layer F.Cu) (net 8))
 (segment (start 83.947 59.182) (end 84.36089 59.182) (width 0.25) (layer F.Cu) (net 8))
 (segment (start 83.82 59.055) (end 83.947 59.182) (width 0.25) (layer F.Cu) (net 8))
 (segment (start 84.2772 58.928) (end 84.582 58.928) (width 0.5) (layer F.Cu) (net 8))
 (segment (start 83.82 58.928) (end 84.2772 58.928) (width 0.5) (layer F.Cu) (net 8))
 (segment (start 83.82 58.928) (end 84.233052 58.928) (width 0.79) (layer F.Cu) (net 8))
 (segment (start 93.28404 59.31408) (end 93.76664 59.31408) (width 0.25) (layer F.Cu) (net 2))
 (segment (start 93.2815 59.8551) (end 93.7641 59.8551) (width 0.25) (layer F.Cu) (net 2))
 (segment (start 93.2688 59.84748) (end 93.02496 59.60364) (width 0.25) (layer F.Cu) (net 2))
 (segment (start 95.77384 59.57824) (end 95.77384 59.58586) (width 0.25) (layer F.Cu) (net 2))
 (segment (start 91.1438 59.57824) (end 95.77384 59.57824) (width 0.25) (layer F.Cu) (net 2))
 (segment (start 91.1438 59.57824) (end 92.89796 59.57824) (width 0.25) (layer F.Cu) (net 2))
 (segment (start 93.01988 59.57824) (end 93.26372 59.3344) (width 0.25) (layer F.Cu) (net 2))
 (segment (start 91.1438 59.57824) (end 92.99956 59.57824) (width 0.25) (layer F.Cu) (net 2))
 (via (at 78.994 57.658) (size 0.8) (drill 0.4) (layers F.Cu B.Cu) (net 7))
 (segment (start 79.062001 57.589999) (end 78.994 57.658) (width 0.79) (layer B.Cu) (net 7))
 (via (at 78.994 60.198) (size 0.8) (drill 0.4) (layers F.Cu B.Cu) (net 7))
 (segment (start 75.967 58.928) (end 78.613 58.928) (width 0.79) (layer F.Cu) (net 7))
 (segment (start 78.994 58.547) (end 78.994 57.658) (width 0.79) (layer F.Cu) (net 7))
 (segment (start 78.613 58.928) (end 78.994 58.547) (width 0.79) (layer F.Cu) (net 7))
 (segment (start 78.994 57.658) (end 78.994 60.198) (width 0.79) (layer F.Cu) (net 7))
 (segment (start 78.994 59.309) (end 78.613 58.928) (width 0.79) (layer F.Cu) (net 7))
 (segment (start 78.994 60.198) (end 78.994 59.309) (width 0.79) (layer F.Cu) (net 7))
 (segment (start 81.026 62.23) (end 78.994 60.198) (width 0.79) (layer B.Cu) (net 7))
 (segment (start 85.217 62.23) (end 81.026 62.23) (width 0.79) (layer B.Cu) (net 7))
 (segment (start 81.026 55.626) (end 78.994 57.658) (width 0.79) (layer B.Cu) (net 7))
 (segment (start 85.217 55.626) (end 81.026 55.626) (width 0.79) (layer B.Cu) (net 7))
 (via (at 86.741 55.626) (size 0.8) (drill 0.4) (layers F.Cu B.Cu) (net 7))
 (segment (start 85.217 55.626) (end 86.741 55.626) (width 0.79) (layer B.Cu) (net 7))
 (segment (start 87.046 55.626) (end 87.884 56.464) (width 0.79) (layer F.Cu) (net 7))
 (segment (start 86.741 55.626) (end 87.046 55.626) (width 0.79) (layer F.Cu) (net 7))
 (via (at 86.741 62.23) (size 0.8) (drill 0.4) (layers F.Cu B.Cu) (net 7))
 (segment (start 85.217 62.23) (end 86.741 62.23) (width 0.79) (layer B.Cu) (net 7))
 (segment (start 87.046 62.23) (end 87.884 61.392) (width 0.79) (layer F.Cu) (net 7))
 (segment (start 86.741 62.23) (end 87.046 62.23) (width 0.79) (layer F.Cu) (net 7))
 (segment (start 100.6841 58.2676) (end 100.6856 58.2691) (width 0.35) (layer F.Cu) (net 3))
 (segment (start 100.6841 59.5884) (end 100.6856 59.5869) (width 0.35) (layer F.Cu) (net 1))
 (segment (start 87.376 59.69) (end 87.56525 59.87925) (width 0.4) (layer F.Cu) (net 5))
 (segment (start 87.63 59.817) (end 87.44075 59.62775) (width 0.4) (layer F.Cu) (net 5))
 (segment (start 88.39329 59.62775) (end 88.39329 59.57824) (width 0.4) (layer F.Cu) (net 5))
 (segment (start 88.20404 59.817) (end 88.39329 59.62775) (width 0.4) (layer F.Cu) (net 5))
 (segment (start 87.884 59.817) (end 88.20404 59.817) (width 0.4) (layer F.Cu) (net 5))
 (segment (start 87.376 58.166) (end 87.56525 57.97675) (width 0.4) (layer F.Cu) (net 6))
 (segment (start 88.39329 58.22825) (end 88.39329 58.27776) (width 0.4) (layer F.Cu) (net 6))
 (segment (start 88.20404 58.039) (end 88.39329 58.22825) (width 0.4) (layer F.Cu) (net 6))
 (segment (start 87.884 58.039) (end 88.20404 58.039) (width 0.4) (layer F.Cu) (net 6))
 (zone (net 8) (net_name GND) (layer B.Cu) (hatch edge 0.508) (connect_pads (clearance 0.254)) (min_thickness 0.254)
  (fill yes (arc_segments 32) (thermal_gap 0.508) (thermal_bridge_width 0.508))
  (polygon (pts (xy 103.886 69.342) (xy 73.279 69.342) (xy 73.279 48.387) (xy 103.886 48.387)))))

